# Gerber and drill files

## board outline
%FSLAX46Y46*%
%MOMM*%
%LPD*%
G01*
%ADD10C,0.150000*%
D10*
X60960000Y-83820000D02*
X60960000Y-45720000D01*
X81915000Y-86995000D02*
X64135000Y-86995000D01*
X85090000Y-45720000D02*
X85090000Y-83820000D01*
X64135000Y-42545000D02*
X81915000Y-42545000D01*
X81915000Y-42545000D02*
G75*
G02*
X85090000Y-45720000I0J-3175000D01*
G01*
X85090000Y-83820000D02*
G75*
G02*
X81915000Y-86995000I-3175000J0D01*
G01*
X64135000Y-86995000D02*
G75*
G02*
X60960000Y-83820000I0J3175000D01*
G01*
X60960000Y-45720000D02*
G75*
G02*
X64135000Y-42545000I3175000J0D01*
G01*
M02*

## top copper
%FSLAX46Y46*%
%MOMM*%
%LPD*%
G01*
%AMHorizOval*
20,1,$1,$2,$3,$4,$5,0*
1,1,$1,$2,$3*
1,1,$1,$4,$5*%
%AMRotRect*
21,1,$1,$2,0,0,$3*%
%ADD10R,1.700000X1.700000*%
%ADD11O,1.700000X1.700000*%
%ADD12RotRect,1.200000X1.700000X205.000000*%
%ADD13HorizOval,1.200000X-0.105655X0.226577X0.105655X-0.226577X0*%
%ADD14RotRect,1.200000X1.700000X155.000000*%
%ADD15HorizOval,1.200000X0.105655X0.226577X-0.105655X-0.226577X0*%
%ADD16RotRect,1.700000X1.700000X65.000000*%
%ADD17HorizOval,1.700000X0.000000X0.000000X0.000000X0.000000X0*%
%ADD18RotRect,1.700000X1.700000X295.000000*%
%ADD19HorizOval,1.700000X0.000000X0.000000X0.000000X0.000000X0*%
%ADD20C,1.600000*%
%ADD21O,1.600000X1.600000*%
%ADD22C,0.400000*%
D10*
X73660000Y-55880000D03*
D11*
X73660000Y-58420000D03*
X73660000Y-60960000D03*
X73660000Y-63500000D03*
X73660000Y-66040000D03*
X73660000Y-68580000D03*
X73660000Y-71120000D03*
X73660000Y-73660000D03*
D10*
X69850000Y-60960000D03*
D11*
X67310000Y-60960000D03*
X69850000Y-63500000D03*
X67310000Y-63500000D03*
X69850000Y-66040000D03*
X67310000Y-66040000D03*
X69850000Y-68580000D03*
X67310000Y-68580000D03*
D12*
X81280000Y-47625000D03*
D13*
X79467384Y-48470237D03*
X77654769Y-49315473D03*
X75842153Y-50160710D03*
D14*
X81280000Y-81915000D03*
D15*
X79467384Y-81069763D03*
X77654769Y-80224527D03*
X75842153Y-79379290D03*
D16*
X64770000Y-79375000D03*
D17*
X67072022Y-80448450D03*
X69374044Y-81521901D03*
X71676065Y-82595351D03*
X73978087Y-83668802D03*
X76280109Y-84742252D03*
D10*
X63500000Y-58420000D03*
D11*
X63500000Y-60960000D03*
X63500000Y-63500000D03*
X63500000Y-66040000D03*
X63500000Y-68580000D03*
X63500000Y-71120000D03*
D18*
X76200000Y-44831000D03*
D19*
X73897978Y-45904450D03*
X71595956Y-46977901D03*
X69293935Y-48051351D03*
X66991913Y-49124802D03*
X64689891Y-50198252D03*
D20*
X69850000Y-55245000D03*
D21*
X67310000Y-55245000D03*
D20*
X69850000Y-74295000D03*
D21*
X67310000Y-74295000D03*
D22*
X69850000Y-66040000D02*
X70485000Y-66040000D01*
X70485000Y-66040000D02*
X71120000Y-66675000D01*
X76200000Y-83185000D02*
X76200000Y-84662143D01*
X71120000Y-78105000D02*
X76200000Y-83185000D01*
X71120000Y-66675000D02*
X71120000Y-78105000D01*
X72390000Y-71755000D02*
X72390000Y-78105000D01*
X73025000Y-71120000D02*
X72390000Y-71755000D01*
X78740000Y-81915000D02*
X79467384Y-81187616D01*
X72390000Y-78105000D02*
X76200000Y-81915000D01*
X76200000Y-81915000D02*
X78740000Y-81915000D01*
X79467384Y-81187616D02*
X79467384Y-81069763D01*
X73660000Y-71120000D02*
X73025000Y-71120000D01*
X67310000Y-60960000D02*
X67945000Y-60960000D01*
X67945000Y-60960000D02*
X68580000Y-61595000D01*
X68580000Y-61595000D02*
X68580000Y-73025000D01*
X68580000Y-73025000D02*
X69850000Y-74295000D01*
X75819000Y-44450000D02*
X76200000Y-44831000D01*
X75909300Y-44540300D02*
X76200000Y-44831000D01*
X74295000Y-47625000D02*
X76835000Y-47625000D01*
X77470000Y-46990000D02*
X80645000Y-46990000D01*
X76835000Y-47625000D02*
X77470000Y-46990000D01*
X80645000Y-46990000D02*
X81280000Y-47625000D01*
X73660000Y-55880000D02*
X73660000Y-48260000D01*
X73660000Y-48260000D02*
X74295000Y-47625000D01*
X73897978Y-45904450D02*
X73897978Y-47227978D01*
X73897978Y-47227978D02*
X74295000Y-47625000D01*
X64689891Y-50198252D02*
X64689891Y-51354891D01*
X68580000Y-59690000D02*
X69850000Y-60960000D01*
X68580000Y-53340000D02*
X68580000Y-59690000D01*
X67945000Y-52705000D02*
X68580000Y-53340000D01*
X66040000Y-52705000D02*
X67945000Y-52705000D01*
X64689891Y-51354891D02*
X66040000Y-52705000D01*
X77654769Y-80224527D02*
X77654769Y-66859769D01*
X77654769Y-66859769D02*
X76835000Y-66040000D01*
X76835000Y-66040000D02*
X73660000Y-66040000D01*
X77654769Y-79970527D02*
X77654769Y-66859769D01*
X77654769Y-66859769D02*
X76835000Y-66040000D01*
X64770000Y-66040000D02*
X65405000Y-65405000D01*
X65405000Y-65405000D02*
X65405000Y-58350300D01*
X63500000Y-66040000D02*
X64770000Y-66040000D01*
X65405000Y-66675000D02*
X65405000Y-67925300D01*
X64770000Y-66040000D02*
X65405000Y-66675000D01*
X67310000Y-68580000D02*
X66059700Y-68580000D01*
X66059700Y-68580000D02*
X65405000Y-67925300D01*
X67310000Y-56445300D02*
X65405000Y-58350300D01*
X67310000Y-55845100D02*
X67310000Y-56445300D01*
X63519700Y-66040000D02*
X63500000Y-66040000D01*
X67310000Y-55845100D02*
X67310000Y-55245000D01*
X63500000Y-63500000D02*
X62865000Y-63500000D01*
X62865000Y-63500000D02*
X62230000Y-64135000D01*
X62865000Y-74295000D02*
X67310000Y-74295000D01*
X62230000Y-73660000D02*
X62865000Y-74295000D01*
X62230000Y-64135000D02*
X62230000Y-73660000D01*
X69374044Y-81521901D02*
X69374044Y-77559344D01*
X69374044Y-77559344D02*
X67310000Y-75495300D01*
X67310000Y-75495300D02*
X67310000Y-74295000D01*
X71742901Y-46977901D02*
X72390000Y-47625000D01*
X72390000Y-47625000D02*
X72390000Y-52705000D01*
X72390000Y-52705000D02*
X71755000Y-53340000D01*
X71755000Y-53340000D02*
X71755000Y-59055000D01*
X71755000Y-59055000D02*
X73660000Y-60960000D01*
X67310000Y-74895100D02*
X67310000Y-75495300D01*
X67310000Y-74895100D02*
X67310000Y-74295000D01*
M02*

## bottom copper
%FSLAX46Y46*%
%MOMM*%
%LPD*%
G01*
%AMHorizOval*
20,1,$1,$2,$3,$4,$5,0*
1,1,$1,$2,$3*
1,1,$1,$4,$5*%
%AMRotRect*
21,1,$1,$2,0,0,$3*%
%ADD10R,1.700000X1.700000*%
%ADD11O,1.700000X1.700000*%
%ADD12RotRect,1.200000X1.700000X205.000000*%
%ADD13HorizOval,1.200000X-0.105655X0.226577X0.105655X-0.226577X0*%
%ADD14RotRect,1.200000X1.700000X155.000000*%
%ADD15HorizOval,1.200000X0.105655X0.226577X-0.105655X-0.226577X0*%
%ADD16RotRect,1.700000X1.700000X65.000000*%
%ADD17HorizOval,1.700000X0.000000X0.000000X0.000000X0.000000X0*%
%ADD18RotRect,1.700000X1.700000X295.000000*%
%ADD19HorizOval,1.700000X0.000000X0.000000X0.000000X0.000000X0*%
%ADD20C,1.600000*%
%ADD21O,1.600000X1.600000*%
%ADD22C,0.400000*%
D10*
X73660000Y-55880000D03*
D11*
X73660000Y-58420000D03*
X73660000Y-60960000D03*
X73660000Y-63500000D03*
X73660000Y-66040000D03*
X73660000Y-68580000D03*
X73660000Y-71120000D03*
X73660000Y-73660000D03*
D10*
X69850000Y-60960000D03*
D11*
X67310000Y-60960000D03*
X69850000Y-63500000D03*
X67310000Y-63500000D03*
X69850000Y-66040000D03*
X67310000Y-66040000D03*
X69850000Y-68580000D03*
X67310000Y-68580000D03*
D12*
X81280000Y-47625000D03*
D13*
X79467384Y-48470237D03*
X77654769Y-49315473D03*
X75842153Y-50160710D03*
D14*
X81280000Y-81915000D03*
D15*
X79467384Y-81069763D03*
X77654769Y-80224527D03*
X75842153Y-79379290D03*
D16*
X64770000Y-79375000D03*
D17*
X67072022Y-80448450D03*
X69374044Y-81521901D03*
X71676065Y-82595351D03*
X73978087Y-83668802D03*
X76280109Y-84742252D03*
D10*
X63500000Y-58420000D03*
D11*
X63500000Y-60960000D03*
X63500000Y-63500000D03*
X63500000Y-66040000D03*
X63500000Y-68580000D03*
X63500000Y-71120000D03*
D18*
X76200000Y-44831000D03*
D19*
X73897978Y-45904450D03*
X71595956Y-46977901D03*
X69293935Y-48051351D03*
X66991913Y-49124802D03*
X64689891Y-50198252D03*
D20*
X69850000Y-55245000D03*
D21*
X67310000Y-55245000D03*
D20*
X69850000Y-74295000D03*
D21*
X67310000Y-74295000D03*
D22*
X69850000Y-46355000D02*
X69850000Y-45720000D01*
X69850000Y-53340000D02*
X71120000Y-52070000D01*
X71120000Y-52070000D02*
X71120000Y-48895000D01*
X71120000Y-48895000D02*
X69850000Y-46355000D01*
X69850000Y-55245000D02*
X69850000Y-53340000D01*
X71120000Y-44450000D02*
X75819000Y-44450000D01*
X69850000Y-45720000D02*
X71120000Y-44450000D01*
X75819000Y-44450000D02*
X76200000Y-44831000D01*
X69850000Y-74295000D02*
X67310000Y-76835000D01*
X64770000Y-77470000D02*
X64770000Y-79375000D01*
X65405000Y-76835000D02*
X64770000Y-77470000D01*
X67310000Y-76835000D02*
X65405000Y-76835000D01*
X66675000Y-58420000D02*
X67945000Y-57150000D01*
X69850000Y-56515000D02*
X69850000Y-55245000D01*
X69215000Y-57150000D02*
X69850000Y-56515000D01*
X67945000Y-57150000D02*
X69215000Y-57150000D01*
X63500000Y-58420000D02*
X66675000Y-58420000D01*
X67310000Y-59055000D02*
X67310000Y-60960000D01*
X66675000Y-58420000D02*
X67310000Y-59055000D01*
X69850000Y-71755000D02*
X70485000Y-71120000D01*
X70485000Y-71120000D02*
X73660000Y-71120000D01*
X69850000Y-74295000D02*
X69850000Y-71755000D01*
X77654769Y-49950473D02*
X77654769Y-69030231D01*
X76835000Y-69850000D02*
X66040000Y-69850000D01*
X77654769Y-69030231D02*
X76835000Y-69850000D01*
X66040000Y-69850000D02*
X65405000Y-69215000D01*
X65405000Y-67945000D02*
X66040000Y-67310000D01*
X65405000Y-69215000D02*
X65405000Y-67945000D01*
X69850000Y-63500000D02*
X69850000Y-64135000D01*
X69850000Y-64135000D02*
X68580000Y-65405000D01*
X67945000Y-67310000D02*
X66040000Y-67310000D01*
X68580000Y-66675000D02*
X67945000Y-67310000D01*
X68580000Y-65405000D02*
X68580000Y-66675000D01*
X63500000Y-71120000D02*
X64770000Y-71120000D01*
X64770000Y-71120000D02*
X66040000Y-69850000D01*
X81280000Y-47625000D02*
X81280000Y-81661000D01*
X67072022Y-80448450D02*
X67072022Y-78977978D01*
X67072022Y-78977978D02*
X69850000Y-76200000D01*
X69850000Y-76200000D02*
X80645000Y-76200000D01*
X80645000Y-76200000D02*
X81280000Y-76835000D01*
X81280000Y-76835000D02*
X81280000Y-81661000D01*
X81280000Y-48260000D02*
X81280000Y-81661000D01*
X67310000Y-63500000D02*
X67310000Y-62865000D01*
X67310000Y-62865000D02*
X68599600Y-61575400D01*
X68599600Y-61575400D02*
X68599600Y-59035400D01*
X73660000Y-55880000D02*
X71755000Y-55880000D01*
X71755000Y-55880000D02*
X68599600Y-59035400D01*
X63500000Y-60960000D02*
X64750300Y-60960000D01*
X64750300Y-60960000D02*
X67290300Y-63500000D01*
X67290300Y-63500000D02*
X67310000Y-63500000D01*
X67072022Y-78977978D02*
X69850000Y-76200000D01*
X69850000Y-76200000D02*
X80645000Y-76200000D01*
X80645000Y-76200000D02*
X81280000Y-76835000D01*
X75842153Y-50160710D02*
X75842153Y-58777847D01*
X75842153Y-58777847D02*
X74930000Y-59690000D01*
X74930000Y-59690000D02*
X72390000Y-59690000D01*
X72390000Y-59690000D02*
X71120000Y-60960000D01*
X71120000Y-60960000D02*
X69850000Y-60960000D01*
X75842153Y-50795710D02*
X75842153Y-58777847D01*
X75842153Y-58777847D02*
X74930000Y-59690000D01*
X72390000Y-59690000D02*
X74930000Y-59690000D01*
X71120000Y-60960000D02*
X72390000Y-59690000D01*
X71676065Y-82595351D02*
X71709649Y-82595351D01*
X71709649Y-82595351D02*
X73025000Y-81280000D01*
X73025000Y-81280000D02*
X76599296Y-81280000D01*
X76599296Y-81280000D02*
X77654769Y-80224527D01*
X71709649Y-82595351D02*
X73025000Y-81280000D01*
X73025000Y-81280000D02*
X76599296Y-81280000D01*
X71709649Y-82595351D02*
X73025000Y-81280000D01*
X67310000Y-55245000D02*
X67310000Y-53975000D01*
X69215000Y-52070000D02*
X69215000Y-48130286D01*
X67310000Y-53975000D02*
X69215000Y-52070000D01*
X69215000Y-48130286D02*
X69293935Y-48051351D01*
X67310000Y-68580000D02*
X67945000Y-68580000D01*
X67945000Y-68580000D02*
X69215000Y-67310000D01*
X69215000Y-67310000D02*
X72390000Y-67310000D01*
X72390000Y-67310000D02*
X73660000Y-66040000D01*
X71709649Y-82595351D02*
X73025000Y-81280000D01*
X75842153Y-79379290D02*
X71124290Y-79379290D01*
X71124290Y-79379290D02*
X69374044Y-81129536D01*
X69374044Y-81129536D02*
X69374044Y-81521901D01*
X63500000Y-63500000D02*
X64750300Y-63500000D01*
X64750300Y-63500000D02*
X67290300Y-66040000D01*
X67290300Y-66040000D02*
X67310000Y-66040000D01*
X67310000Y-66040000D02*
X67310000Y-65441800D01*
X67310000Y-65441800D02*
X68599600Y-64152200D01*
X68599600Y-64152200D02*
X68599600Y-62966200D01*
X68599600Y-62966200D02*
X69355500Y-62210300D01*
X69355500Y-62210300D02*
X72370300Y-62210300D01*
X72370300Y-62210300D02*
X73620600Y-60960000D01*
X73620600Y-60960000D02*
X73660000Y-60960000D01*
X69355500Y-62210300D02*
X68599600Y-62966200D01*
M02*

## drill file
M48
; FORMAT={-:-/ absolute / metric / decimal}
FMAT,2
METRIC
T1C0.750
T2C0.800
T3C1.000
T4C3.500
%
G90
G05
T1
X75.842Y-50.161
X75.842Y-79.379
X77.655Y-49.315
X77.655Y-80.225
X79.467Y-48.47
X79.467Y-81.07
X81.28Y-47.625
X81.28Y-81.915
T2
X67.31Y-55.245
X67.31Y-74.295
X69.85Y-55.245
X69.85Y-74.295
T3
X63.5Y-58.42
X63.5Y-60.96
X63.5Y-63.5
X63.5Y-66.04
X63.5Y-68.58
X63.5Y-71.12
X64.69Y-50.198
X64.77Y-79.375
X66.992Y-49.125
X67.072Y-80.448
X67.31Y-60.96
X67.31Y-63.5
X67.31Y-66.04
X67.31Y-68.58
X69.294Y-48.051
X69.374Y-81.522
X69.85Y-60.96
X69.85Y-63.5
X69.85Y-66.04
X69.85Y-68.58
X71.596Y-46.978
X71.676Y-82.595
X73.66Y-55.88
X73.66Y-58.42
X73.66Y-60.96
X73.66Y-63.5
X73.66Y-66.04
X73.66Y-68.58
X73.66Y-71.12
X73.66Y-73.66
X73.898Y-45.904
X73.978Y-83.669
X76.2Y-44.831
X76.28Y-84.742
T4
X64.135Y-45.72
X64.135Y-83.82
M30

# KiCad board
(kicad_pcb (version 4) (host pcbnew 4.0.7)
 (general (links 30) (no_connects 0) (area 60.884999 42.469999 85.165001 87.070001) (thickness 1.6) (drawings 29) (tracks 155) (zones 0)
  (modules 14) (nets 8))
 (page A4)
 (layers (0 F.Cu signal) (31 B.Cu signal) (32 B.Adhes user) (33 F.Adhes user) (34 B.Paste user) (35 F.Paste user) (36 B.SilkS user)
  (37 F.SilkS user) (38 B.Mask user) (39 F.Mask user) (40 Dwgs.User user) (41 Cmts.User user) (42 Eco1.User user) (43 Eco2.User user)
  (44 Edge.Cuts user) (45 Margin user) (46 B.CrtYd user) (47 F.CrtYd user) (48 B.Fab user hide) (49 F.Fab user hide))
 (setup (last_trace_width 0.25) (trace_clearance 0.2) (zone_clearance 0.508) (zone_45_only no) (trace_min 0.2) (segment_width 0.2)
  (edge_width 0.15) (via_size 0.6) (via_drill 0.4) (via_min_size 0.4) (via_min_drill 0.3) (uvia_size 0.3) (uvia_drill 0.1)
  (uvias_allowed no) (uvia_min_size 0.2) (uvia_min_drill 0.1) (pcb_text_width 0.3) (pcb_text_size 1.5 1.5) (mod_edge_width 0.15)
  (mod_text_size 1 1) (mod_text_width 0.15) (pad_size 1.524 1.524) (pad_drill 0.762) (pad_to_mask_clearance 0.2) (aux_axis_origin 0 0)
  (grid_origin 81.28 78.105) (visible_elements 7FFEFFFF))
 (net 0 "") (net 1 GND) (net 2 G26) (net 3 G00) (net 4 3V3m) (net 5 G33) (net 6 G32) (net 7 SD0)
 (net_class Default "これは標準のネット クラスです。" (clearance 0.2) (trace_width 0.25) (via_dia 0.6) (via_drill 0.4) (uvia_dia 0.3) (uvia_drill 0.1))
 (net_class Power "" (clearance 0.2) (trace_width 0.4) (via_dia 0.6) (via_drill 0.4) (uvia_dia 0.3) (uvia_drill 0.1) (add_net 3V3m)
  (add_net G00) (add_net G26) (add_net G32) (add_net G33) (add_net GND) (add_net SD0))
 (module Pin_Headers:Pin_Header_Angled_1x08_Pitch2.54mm (layer F.Cu) (at 73.66 55.88)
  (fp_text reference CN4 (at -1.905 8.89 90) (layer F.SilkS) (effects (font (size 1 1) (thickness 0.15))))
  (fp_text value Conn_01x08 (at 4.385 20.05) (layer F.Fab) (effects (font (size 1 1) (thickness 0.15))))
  (pad 1 thru_hole rect (at 0 0) (size 1.7 1.7) (drill 1) (layers *.Cu *.Mask) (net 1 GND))
  (pad 2 thru_hole oval (at 0 2.54) (size 1.7 1.7) (drill 1) (layers *.Cu *.Mask))
  (pad 3 thru_hole oval (at 0 5.08) (size 1.7 1.7) (drill 1) (layers *.Cu *.Mask) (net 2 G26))
  (pad 4 thru_hole oval (at 0 7.62) (size 1.7 1.7) (drill 1) (layers *.Cu *.Mask))
  (pad 5 thru_hole oval (at 0 10.16) (size 1.7 1.7) (drill 1) (layers *.Cu *.Mask) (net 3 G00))
  (pad 6 thru_hole oval (at 0 12.7) (size 1.7 1.7) (drill 1) (layers *.Cu *.Mask))
  (pad 7 thru_hole oval (at 0 15.24) (size 1.7 1.7) (drill 1) (layers *.Cu *.Mask) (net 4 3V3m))
  (pad 8 thru_hole oval (at 0 17.78) (size 1.7 1.7) (drill 1) (layers *.Cu *.Mask)))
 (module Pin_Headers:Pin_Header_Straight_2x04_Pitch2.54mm (layer B.Cu) (at 69.85 60.96 180)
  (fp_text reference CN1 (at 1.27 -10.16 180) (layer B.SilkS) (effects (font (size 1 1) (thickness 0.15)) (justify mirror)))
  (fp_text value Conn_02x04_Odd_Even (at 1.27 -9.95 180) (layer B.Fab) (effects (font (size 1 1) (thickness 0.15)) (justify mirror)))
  (pad 1 thru_hole rect (at 0 0 180) (size 1.7 1.7) (drill 1) (layers *.Cu *.Mask) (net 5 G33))
  (pad 2 thru_hole oval (at 2.54 0 180) (size 1.7 1.7) (drill 1) (layers *.Cu *.Mask) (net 4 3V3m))
  (pad 3 thru_hole oval (at 0 -2.54 180) (size 1.7 1.7) (drill 1) (layers *.Cu *.Mask) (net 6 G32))
  (pad 4 thru_hole oval (at 2.54 -2.54 180) (size 1.7 1.7) (drill 1) (layers *.Cu *.Mask) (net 1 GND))
  (pad 5 thru_hole oval (at 0 -5.08 180) (size 1.7 1.7) (drill 1) (layers *.Cu *.Mask) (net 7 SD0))
  (pad 6 thru_hole oval (at 2.54 -5.08 180) (size 1.7 1.7) (drill 1) (layers *.Cu *.Mask) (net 2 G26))
  (pad 7 thru_hole oval (at 0 -7.62 180) (size 1.7 1.7) (drill 1) (layers *.Cu *.Mask))
  (pad 8 thru_hole oval (at 2.54 -7.62 180) (size 1.7 1.7) (drill 1) (layers *.Cu *.Mask) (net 3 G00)))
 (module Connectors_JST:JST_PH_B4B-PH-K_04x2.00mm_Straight (layer F.Cu) (at 81.28 47.625 205)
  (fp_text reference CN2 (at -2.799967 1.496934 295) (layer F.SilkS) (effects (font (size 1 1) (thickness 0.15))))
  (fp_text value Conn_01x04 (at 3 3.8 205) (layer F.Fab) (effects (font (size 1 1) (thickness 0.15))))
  (pad 1 thru_hole rect (at 0 0 205) (size 1.2 1.7) (drill 0.75) (layers *.Cu *.Mask) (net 1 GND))
  (pad 2 thru_hole oval (at 2 0 205) (size 1.2 1.7) (drill 0.75) (layers *.Cu *.Mask))
  (pad 3 thru_hole oval (at 4 0 205) (size 1.2 1.7) (drill 0.75) (layers *.Cu *.Mask) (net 6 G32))
  (pad 4 thru_hole oval (at 6 0 205) (size 1.2 1.7) (drill 0.75) (layers *.Cu *.Mask) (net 5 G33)))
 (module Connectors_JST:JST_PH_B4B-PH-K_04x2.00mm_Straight (layer F.Cu) (at 81.28 81.915 155)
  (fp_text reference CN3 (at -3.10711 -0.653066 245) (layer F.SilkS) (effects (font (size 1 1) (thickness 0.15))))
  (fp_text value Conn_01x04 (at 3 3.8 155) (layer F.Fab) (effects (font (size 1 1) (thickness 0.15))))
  (pad 1 thru_hole rect (at 0 0 155) (size 1.2 1.7) (drill 0.75) (layers *.Cu *.Mask) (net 1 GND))
  (pad 2 thru_hole oval (at 2 0 155) (size 1.2 1.7) (drill 0.75) (layers *.Cu *.Mask) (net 4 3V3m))
  (pad 3 thru_hole oval (at 4 0 155) (size 1.2 1.7) (drill 0.75) (layers *.Cu *.Mask) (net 3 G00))
  (pad 4 thru_hole oval (at 6 0 155) (size 1.2 1.7) (drill 0.75) (layers *.Cu *.Mask) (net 2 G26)))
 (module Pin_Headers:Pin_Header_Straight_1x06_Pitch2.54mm (layer F.Cu) (at 64.77 79.375 65)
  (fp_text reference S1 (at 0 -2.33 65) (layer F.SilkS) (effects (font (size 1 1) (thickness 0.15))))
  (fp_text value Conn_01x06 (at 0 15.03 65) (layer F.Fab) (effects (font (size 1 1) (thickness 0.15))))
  (pad 1 thru_hole rect (at 0 0 65) (size 1.7 1.7) (drill 1) (layers *.Cu *.Mask) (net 4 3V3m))
  (pad 2 thru_hole oval (at 0 2.54 65) (size 1.7 1.7) (drill 1) (layers *.Cu *.Mask) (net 1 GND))
  (pad 3 thru_hole oval (at 0 5.08 65) (size 1.7 1.7) (drill 1) (layers *.Cu *.Mask) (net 2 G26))
  (pad 4 thru_hole oval (at 0 7.62 65) (size 1.7 1.7) (drill 1) (layers *.Cu *.Mask) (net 3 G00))
  (pad 5 thru_hole oval (at 0 10.16 65) (size 1.7 1.7) (drill 1) (layers *.Cu *.Mask))
  (pad 6 thru_hole oval (at 0 12.7 65) (size 1.7 1.7) (drill 1) (layers *.Cu *.Mask) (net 7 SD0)))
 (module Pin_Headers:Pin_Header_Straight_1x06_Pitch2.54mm (layer F.Cu) (at 63.5 58.42)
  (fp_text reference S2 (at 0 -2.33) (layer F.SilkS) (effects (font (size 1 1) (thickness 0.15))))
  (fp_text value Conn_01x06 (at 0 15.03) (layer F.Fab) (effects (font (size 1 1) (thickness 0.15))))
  (pad 1 thru_hole rect (at 0 0) (size 1.7 1.7) (drill 1) (layers *.Cu *.Mask) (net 4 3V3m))
  (pad 2 thru_hole oval (at 0 2.54) (size 1.7 1.7) (drill 1) (layers *.Cu *.Mask) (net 1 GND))
  (pad 3 thru_hole oval (at 0 5.08) (size 1.7 1.7) (drill 1) (layers *.Cu *.Mask) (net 2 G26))
  (pad 4 thru_hole oval (at 0 7.62) (size 1.7 1.7) (drill 1) (layers *.Cu *.Mask) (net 3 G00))
  (pad 5 thru_hole oval (at 0 10.16) (size 1.7 1.7) (drill 1) (layers *.Cu *.Mask))
  (pad 6 thru_hole oval (at 0 12.7) (size 1.7 1.7) (drill 1) (layers *.Cu *.Mask) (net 6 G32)))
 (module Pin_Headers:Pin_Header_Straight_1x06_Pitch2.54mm (layer F.Cu) (at 76.2 44.831 295)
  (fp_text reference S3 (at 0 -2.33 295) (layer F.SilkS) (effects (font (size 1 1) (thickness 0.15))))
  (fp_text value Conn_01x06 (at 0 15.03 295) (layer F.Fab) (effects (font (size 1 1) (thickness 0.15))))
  (pad 1 thru_hole rect (at 0 0 295) (size 1.7 1.7) (drill 1) (layers *.Cu *.Mask) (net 4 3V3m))
  (pad 2 thru_hole oval (at 0 2.54 295) (size 1.7 1.7) (drill 1) (layers *.Cu *.Mask) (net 1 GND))
  (pad 3 thru_hole oval (at 0 5.08 295) (size 1.7 1.7) (drill 1) (layers *.Cu *.Mask) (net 2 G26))
  (pad 4 thru_hole oval (at 0 7.62 295) (size 1.7 1.7) (drill 1) (layers *.Cu *.Mask) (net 3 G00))
  (pad 5 thru_hole oval (at 0 10.16 295) (size 1.7 1.7) (drill 1) (layers *.Cu *.Mask))
  (pad 6 thru_hole oval (at 0 12.7 295) (size 1.7 1.7) (drill 1) (layers *.Cu *.Mask) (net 5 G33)))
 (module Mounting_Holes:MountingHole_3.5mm (layer F.Cu) (at 64.135 45.72)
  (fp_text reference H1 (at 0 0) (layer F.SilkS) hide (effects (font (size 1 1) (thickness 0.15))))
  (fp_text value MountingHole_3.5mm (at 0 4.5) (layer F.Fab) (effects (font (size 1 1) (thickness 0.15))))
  (pad 1 np_thru_hole circle (at 0 0) (size 3.5 3.5) (drill 3.5) (layers *.Cu *.Mask)))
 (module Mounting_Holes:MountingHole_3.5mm (layer F.Cu) (at 64.135 83.82)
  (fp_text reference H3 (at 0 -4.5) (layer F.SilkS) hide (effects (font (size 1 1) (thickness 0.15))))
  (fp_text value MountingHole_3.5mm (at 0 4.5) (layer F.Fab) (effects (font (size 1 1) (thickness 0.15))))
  (pad 1 np_thru_hole circle (at 0 0) (size 3.5 3.5) (drill 3.5) (layers *.Cu *.Mask)))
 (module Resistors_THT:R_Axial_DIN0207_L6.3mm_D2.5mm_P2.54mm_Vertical (layer F.Cu) (at 69.85 55.245 180)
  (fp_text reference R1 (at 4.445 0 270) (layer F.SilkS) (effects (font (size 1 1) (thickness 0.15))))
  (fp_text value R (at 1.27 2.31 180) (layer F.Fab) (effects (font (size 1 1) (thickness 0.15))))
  (pad 1 thru_hole circle (at 0 0 180) (size 1.6 1.6) (drill 0.8) (layers *.Cu *.Mask) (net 4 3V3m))
  (pad 2 thru_hole oval (at 2.54 0 180) (size 1.6 1.6) (drill 0.8) (layers *.Cu *.Mask) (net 3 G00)))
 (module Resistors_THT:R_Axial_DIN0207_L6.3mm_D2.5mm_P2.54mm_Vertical (layer F.Cu) (at 69.85 74.295 180)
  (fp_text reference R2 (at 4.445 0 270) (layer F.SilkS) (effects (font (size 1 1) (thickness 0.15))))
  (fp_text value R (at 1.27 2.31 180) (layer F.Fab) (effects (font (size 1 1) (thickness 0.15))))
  (pad 1 thru_hole circle (at 0 0 180) (size 1.6 1.6) (drill 0.8) (layers *.Cu *.Mask) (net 4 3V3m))
  (pad 2 thru_hole oval (at 2.54 0 180) (size 1.6 1.6) (drill 0.8) (layers *.Cu *.Mask) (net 2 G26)))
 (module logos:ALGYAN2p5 (layer B.Cu) (at 80.645 64.135 270)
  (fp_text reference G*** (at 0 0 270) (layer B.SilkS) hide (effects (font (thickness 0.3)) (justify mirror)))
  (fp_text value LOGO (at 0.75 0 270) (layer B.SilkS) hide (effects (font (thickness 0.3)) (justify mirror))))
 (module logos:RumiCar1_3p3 (layer B.Cu) (at 77.1525 58.7375 270)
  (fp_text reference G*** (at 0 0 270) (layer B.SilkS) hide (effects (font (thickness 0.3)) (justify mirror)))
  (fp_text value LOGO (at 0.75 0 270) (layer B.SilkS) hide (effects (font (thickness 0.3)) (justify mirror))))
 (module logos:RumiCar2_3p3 (layer B.Cu) (at 77.1525 66.3575 270)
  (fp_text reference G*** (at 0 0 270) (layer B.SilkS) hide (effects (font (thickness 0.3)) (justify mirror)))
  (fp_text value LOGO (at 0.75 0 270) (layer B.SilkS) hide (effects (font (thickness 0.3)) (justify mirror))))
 (gr_line (start 60.96 83.82) (end 60.96 45.72) (angle 90) (layer Edge.Cuts) (width 0.15))
 (gr_line (start 81.915 86.995) (end 64.135 86.995) (angle 90) (layer Edge.Cuts) (width 0.15))
 (gr_line (start 85.09 45.72) (end 85.09 83.82) (angle 90) (layer Edge.Cuts) (width 0.15))
 (gr_line (start 64.135 42.545) (end 81.915 42.545) (angle 90) (layer Edge.Cuts) (width 0.15))
 (gr_arc (start 81.915 45.72) (end 81.915 42.545) (angle 90) (layer Edge.Cuts) (width 0.15))
 (gr_arc (start 81.915 83.82) (end 85.09 83.82) (angle 90) (layer Edge.Cuts) (width 0.15))
 (gr_arc (start 64.135 83.82) (end 64.135 86.995) (angle 90) (layer Edge.Cuts) (width 0.15))
 (gr_arc (start 64.135 45.72) (end 60.96 45.72) (angle 90) (layer Edge.Cuts) (width 0.15))
 (segment (start 69.85 66.04) (end 70.485 66.04) (width 0.4) (layer F.Cu) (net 7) (status 30))
 (segment (start 70.485 66.04) (end 71.12 66.675) (width 0.4) (layer F.Cu) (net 7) (status 10))
 (segment (start 76.2 83.185) (end 76.2 84.662143) (width 0.4) (layer F.Cu) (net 7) (status 20))
 (segment (start 71.12 78.105) (end 76.2 83.185) (width 0.4) (layer F.Cu) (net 7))
 (segment (start 71.12 66.675) (end 71.12 78.105) (width 0.4) (layer F.Cu) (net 7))
 (segment (start 72.39 71.755) (end 72.39 78.105) (width 0.4) (layer F.Cu) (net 4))
 (segment (start 73.025 71.12) (end 72.39 71.755) (width 0.4) (layer F.Cu) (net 4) (status 10))
 (segment (start 78.74 81.915) (end 79.467384 81.187616) (width 0.4) (layer F.Cu) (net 4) (status 20))
 (segment (start 72.39 78.105) (end 76.2 81.915) (width 0.4) (layer F.Cu) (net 4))
 (segment (start 76.2 81.915) (end 78.74 81.915) (width 0.4) (layer F.Cu) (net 4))
 (segment (start 79.467384 81.187616) (end 79.467384 81.069763) (width 0.4) (layer F.Cu) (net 4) (status 30))
 (segment (start 69.85 46.355) (end 69.85 45.72) (width 0.4) (layer B.Cu) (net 4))
 (segment (start 69.85 53.34) (end 71.12 52.07) (width 0.4) (layer B.Cu) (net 4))
 (segment (start 71.12 52.07) (end 71.12 48.895) (width 0.4) (layer B.Cu) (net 4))
 (segment (start 71.12 48.895) (end 69.85 46.355) (width 0.4) (layer B.Cu) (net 4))
 (segment (start 69.85 55.245) (end 69.85 53.34) (width 0.4) (layer B.Cu) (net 4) (status 10))
 (segment (start 71.12 44.45) (end 75.819 44.45) (width 0.4) (layer B.Cu) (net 4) (status 20))
 (segment (start 69.85 45.72) (end 71.12 44.45) (width 0.4) (layer B.Cu) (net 4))
 (segment (start 75.819 44.45) (end 76.2 44.831) (width 0.4) (layer B.Cu) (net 4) (status 30))
 (segment (start 73.66 71.12) (end 73.025 71.12) (width 0.4) (layer F.Cu) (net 4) (status 30))
 (segment (start 69.85 74.295) (end 67.31 76.835) (width 0.4) (layer B.Cu) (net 4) (status 10))
 (segment (start 64.77 77.47) (end 64.77 79.375) (width 0.4) (layer B.Cu) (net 4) (status 20))
 (segment (start 65.405 76.835) (end 64.77 77.47) (width 0.4) (layer B.Cu) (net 4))
 (segment (start 67.31 76.835) (end 65.405 76.835) (width 0.4) (layer B.Cu) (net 4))
 (segment (start 67.31 60.96) (end 67.945 60.96) (width 0.4) (layer F.Cu) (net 4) (status 30))
 (segment (start 67.945 60.96) (end 68.58 61.595) (width 0.4) (layer F.Cu) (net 4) (status 10))
 (segment (start 68.58 61.595) (end 68.58 73.025) (width 0.4) (layer F.Cu) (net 4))
 (segment (start 68.58 73.025) (end 69.85 74.295) (width 0.4) (layer F.Cu) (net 4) (status 20))
 (segment (start 66.675 58.42) (end 67.945 57.15) (width 0.4) (layer B.Cu) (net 4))
 (segment (start 69.85 56.515) (end 69.85 55.245) (width 0.4) (layer B.Cu) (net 4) (status 20))
 (segment (start 69.215 57.15) (end 69.85 56.515) (width 0.4) (layer B.Cu) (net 4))
 (segment (start 67.945 57.15) (end 69.215 57.15) (width 0.4) (layer B.Cu) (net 4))
 (segment (start 63.5 58.42) (end 66.675 58.42) (width 0.4) (layer B.Cu) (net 4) (status 10))
 (segment (start 67.31 59.055) (end 67.31 60.96) (width 0.4) (layer B.Cu) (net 4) (status 20))
 (segment (start 66.675 58.42) (end 67.31 59.055) (width 0.4) (layer B.Cu) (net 4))
 (segment (start 69.85 71.755) (end 70.485 71.12) (width 0.4) (layer B.Cu) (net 4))
 (segment (start 70.485 71.12) (end 73.66 71.12) (width 0.4) (layer B.Cu) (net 4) (status 20))
 (segment (start 69.85 74.295) (end 69.85 71.755) (width 0.4) (layer B.Cu) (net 4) (status 10))
 (segment (start 75.819 44.45) (end 76.2 44.831) (width 0.4) (layer F.Cu) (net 4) (status 30))
 (segment (start 75.9093 44.5403) (end 76.2 44.831) (width 0.4) (layer F.Cu) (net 4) (status 30))
 (segment (start 77.654769 49.950473) (end 77.654769 69.030231) (width 0.4) (layer B.Cu) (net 6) (status 10))
 (segment (start 76.835 69.85) (end 66.04 69.85) (width 0.4) (layer B.Cu) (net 6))
 (segment (start 77.654769 69.030231) (end 76.835 69.85) (width 0.4) (layer B.Cu) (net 6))
 (segment (start 66.04 69.85) (end 65.405 69.215) (width 0.4) (layer B.Cu) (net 6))
 (segment (start 65.405 67.945) (end 66.04 67.31) (width 0.4) (layer B.Cu) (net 6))
 (segment (start 65.405 69.215) (end 65.405 67.945) (width 0.4) (layer B.Cu) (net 6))
 (segment (start 69.85 63.5) (end 69.85 64.135) (width 0.4) (layer B.Cu) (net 6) (status 30))
 (segment (start 69.85 64.135) (end 68.58 65.405) (width 0.4) (layer B.Cu) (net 6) (status 10))
 (segment (start 67.945 67.31) (end 66.04 67.31) (width 0.4) (layer B.Cu) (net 6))
 (segment (start 68.58 66.675) (end 67.945 67.31) (width 0.4) (layer B.Cu) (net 6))
 (segment (start 68.58 65.405) (end 68.58 66.675) (width 0.4) (layer B.Cu) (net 6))
 (segment (start 63.5 71.12) (end 64.77 71.12) (width 0.4) (layer B.Cu) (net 6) (status 10))
 (segment (start 64.77 71.12) (end 66.04 69.85) (width 0.4) (layer B.Cu) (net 6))
 (segment (start 81.28 47.625) (end 81.28 81.661) (width 0.4) (layer B.Cu) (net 1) (status 30))
 (segment (start 74.295 47.625) (end 76.835 47.625) (width 0.4) (layer F.Cu) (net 1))
 (segment (start 77.47 46.99) (end 80.645 46.99) (width 0.4) (layer F.Cu) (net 1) (status 20))
 (segment (start 76.835 47.625) (end 77.47 46.99) (width 0.4) (layer F.Cu) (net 1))
 (segment (start 80.645 46.99) (end 81.28 47.625) (width 0.4) (layer F.Cu) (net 1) (status 30))
 (segment (start 67.072022 80.44845) (end 67.072022 78.977978) (width 0.4) (layer B.Cu) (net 1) (status 10))
 (segment (start 67.072022 78.977978) (end 69.85 76.2) (width 0.4) (layer B.Cu) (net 1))
 (segment (start 69.85 76.2) (end 80.645 76.2) (width 0.4) (layer B.Cu) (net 1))
 (segment (start 80.645 76.2) (end 81.28 76.835) (width 0.4) (layer B.Cu) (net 1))
 (segment (start 81.28 76.835) (end 81.28 81.661) (width 0.4) (layer B.Cu) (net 1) (status 20))
 (segment (start 81.28 48.26) (end 81.28 81.661) (width 0.4) (layer B.Cu) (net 1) (status 30))
 (segment (start 73.66 55.88) (end 73.66 48.26) (width 0.4) (layer F.Cu) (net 1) (status 10))
 (segment (start 73.66 48.26) (end 74.295 47.625) (width 0.4) (layer F.Cu) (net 1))
 (segment (start 73.897978 45.90445) (end 73.897978 47.227978) (width 0.4) (layer F.Cu) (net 1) (status 10))
 (segment (start 73.897978 47.227978) (end 74.295 47.625) (width 0.4) (layer F.Cu) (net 1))
 (segment (start 67.31 63.5) (end 67.31 62.865) (width 0.4) (layer B.Cu) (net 1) (status 30))
 (segment (start 67.31 62.865) (end 68.5996 61.5754) (width 0.4) (layer B.Cu) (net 1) (status 10))
 (segment (start 68.5996 61.5754) (end 68.5996 59.0354) (width 0.4) (layer B.Cu) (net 1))
 (segment (start 73.66 55.88) (end 71.755 55.88) (width 0.4) (layer B.Cu) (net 1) (status 10))
 (segment (start 71.755 55.88) (end 68.5996 59.0354) (width 0.4) (layer B.Cu) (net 1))
 (segment (start 63.5 60.96) (end 64.7503 60.96) (width 0.4) (layer B.Cu) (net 1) (status 10))
 (segment (start 64.7503 60.96) (end 67.2903 63.5) (width 0.4) (layer B.Cu) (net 1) (status 20))
 (segment (start 67.2903 63.5) (end 67.31 63.5) (width 0.4) (layer B.Cu) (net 1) (status 30))
 (segment (start 67.072022 78.977978) (end 69.85 76.2) (width 0.4) (layer B.Cu) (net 1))
 (segment (start 69.85 76.2) (end 80.645 76.2) (width 0.4) (layer B.Cu) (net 1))
 (segment (start 80.645 76.2) (end 81.28 76.835) (width 0.4) (layer B.Cu) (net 1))
 (segment (start 75.842153 50.16071) (end 75.842153 58.777847) (width 0.4) (layer B.Cu) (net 5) (status 10))
 (segment (start 75.842153 58.777847) (end 74.93 59.69) (width 0.4) (layer B.Cu) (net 5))
 (segment (start 74.93 59.69) (end 72.39 59.69) (width 0.4) (layer B.Cu) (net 5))
 (segment (start 72.39 59.69) (end 71.12 60.96) (width 0.4) (layer B.Cu) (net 5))
 (segment (start 71.12 60.96) (end 69.85 60.96) (width 0.4) (layer B.Cu) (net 5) (status 20))
 (segment (start 75.842153 50.79571) (end 75.842153 58.777847) (width 0.4) (layer B.Cu) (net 5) (status 10))
 (segment (start 75.842153 58.777847) (end 74.93 59.69) (width 0.4) (layer B.Cu) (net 5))
 (segment (start 72.39 59.69) (end 74.93 59.69) (width 0.4) (layer B.Cu) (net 5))
 (segment (start 71.12 60.96) (end 72.39 59.69) (width 0.4) (layer B.Cu) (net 5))
 (segment (start 64.689891 50.198252) (end 64.689891 51.354891) (width 0.4) (layer F.Cu) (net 5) (status 10))
 (segment (start 68.58 59.69) (end 69.85 60.96) (width 0.4) (layer F.Cu) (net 5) (status 20))
 (segment (start 68.58 53.34) (end 68.58 59.69) (width 0.4) (layer F.Cu) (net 5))
 (segment (start 67.945 52.705) (end 68.58 53.34) (width 0.4) (layer F.Cu) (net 5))
 (segment (start 66.04 52.705) (end 67.945 52.705) (width 0.4) (layer F.Cu) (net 5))
 (segment (start 64.689891 51.354891) (end 66.04 52.705) (width 0.4) (layer F.Cu) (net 5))
 (segment (start 71.676065 82.595351) (end 71.709649 82.595351) (width 0.4) (layer B.Cu) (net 3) (status 30))
 (segment (start 71.709649 82.595351) (end 73.025 81.28) (width 0.4) (layer B.Cu) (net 3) (status 10))
 (segment (start 73.025 81.28) (end 76.599296 81.28) (width 0.4) (layer B.Cu) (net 3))
 (segment (start 76.599296 81.28) (end 77.654769 80.224527) (width 0.4) (layer B.Cu) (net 3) (status 20))
 (segment (start 77.654769 80.224527) (end 77.654769 66.859769) (width 0.4) (layer F.Cu) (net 3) (status 10))
 (segment (start 77.654769 66.859769) (end 76.835 66.04) (width 0.4) (layer F.Cu) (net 3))
 (segment (start 76.835 66.04) (end 73.66 66.04) (width 0.4) (layer F.Cu) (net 3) (status 20))
 (segment (start 71.709649 82.595351) (end 73.025 81.28) (width 0.4) (layer B.Cu) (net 3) (status 10))
 (segment (start 73.025 81.28) (end 76.599296 81.28) (width 0.4) (layer B.Cu) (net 3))
 (segment (start 77.654769 79.970527) (end 77.654769 66.859769) (width 0.4) (layer F.Cu) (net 3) (status 10))
 (segment (start 77.654769 66.859769) (end 76.835 66.04) (width 0.4) (layer F.Cu) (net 3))
 (segment (start 71.709649 82.595351) (end 73.025 81.28) (width 0.4) (layer B.Cu) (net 3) (status 10))
 (segment (start 67.31 55.245) (end 67.31 53.975) (width 0.4) (layer B.Cu) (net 3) (status 10))
 (segment (start 69.215 52.07) (end 69.215 48.130286) (width 0.4) (layer B.Cu) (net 3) (status 20))
 (segment (start 67.31 53.975) (end 69.215 52.07) (width 0.4) (layer B.Cu) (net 3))
 (segment (start 69.215 48.130286) (end 69.293935 48.051351) (width 0.4) (layer B.Cu) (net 3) (status 30))
 (segment (start 64.77 66.04) (end 65.405 65.405) (width 0.4) (layer F.Cu) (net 3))
 (segment (start 65.405 65.405) (end 65.405 58.3503) (width 0.4) (layer F.Cu) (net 3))
 (segment (start 63.5 66.04) (end 64.77 66.04) (width 0.4) (layer F.Cu) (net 3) (status 10))
 (segment (start 65.405 66.675) (end 65.405 67.9253) (width 0.4) (layer F.Cu) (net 3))
 (segment (start 64.77 66.04) (end 65.405 66.675) (width 0.4) (layer F.Cu) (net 3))
 (segment (start 67.31 68.58) (end 67.945 68.58) (width 0.4) (layer B.Cu) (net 3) (status 30))
 (segment (start 67.945 68.58) (end 69.215 67.31) (width 0.4) (layer B.Cu) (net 3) (status 10))
 (segment (start 69.215 67.31) (end 72.39 67.31) (width 0.4) (layer B.Cu) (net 3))
 (segment (start 72.39 67.31) (end 73.66 66.04) (width 0.4) (layer B.Cu) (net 3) (status 20))
 (segment (start 71.709649 82.595351) (end 73.025 81.28) (width 0.4) (layer B.Cu) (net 3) (status 10))
 (segment (start 67.31 68.58) (end 66.0597 68.58) (width 0.4) (layer F.Cu) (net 3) (status 10))
 (segment (start 66.0597 68.58) (end 65.405 67.9253) (width 0.4) (layer F.Cu) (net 3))
 (segment (start 67.31 56.4453) (end 65.405 58.3503) (width 0.4) (layer F.Cu) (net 3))
 (segment (start 67.31 55.8451) (end 67.31 56.4453) (width 0.4) (layer F.Cu) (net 3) (status 10))
 (segment (start 63.5197 66.04) (end 63.5 66.04) (width 0.4) (layer F.Cu) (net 3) (status 30))
 (segment (start 67.31 55.8451) (end 67.31 55.245) (width 0.4) (layer F.Cu) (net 3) (status 30))
 (segment (start 75.842153 79.37929) (end 71.12429 79.37929) (width 0.4) (layer B.Cu) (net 2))
 (segment (start 71.12429 79.37929) (end 69.374044 81.129536) (width 0.4) (layer B.Cu) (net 2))
 (segment (start 69.374044 81.129536) (end 69.374044 81.521901) (width 0.4) (layer B.Cu) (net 2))
 (segment (start 63.5 63.5) (end 62.865 63.5) (width 0.4) (layer F.Cu) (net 2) (status 30))
 (segment (start 62.865 63.5) (end 62.23 64.135) (width 0.4) (layer F.Cu) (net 2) (status 10))
 (segment (start 62.865 74.295) (end 67.31 74.295) (width 0.4) (layer F.Cu) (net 2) (status 20))
 (segment (start 62.23 73.66) (end 62.865 74.295) (width 0.4) (layer F.Cu) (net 2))
 (segment (start 62.23 64.135) (end 62.23 73.66) (width 0.4) (layer F.Cu) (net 2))
 (segment (start 63.5 63.5) (end 64.7503 63.5) (width 0.4) (layer B.Cu) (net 2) (status 10))
 (segment (start 64.7503 63.5) (end 67.2903 66.04) (width 0.4) (layer B.Cu) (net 2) (status 20))
 (segment (start 67.2903 66.04) (end 67.31 66.04) (width 0.4) (layer B.Cu) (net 2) (status 30))
 (segment (start 67.31 66.04) (end 67.31 65.4418) (width 0.4) (layer B.Cu) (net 2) (status 30))
 (segment (start 67.31 65.4418) (end 68.5996 64.1522) (width 0.4) (layer B.Cu) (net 2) (status 10))
 (segment (start 68.5996 64.1522) (end 68.5996 62.9662) (width 0.4) (layer B.Cu) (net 2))
 (segment (start 68.5996 62.9662) (end 69.3555 62.2103) (width 0.4) (layer B.Cu) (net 2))
 (segment (start 69.3555 62.2103) (end 72.3703 62.2103) (width 0.4) (layer B.Cu) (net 2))
 (segment (start 72.3703 62.2103) (end 73.6206 60.96) (width 0.4) (layer B.Cu) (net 2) (status 20))
 (segment (start 73.6206 60.96) (end 73.66 60.96) (width 0.4) (layer B.Cu) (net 2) (status 30))
 (segment (start 69.374044 81.521901) (end 69.374044 77.559344) (width 0.4) (layer F.Cu) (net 2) (status 10))
 (segment (start 69.374044 77.559344) (end 67.31 75.4953) (width 0.4) (layer F.Cu) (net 2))
 (segment (start 67.31 75.4953) (end 67.31 74.295) (width 0.4) (layer F.Cu) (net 2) (status 20))
 (segment (start 71.742901 46.977901) (end 72.39 47.625) (width 0.4) (layer F.Cu) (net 2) (status 10))
 (segment (start 72.39 47.625) (end 72.39 52.705) (width 0.4) (layer F.Cu) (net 2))
 (segment (start 72.39 52.705) (end 71.755 53.34) (width 0.4) (layer F.Cu) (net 2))
 (segment (start 71.755 53.34) (end 71.755 59.055) (width 0.4) (layer F.Cu) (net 2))
 (segment (start 71.755 59.055) (end 73.66 60.96) (width 0.4) (layer F.Cu) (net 2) (status 20))
 (segment (start 69.3555 62.2103) (end 68.5996 62.9662) (width 0.4) (layer B.Cu) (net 2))
 (segment (start 67.31 74.8951) (end 67.31 75.4953) (width 0.4) (layer F.Cu) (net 2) (status 10))
 (segment (start 67.31 74.8951) (end 67.31 74.295) (width 0.4) (layer F.Cu) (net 2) (status 30)))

